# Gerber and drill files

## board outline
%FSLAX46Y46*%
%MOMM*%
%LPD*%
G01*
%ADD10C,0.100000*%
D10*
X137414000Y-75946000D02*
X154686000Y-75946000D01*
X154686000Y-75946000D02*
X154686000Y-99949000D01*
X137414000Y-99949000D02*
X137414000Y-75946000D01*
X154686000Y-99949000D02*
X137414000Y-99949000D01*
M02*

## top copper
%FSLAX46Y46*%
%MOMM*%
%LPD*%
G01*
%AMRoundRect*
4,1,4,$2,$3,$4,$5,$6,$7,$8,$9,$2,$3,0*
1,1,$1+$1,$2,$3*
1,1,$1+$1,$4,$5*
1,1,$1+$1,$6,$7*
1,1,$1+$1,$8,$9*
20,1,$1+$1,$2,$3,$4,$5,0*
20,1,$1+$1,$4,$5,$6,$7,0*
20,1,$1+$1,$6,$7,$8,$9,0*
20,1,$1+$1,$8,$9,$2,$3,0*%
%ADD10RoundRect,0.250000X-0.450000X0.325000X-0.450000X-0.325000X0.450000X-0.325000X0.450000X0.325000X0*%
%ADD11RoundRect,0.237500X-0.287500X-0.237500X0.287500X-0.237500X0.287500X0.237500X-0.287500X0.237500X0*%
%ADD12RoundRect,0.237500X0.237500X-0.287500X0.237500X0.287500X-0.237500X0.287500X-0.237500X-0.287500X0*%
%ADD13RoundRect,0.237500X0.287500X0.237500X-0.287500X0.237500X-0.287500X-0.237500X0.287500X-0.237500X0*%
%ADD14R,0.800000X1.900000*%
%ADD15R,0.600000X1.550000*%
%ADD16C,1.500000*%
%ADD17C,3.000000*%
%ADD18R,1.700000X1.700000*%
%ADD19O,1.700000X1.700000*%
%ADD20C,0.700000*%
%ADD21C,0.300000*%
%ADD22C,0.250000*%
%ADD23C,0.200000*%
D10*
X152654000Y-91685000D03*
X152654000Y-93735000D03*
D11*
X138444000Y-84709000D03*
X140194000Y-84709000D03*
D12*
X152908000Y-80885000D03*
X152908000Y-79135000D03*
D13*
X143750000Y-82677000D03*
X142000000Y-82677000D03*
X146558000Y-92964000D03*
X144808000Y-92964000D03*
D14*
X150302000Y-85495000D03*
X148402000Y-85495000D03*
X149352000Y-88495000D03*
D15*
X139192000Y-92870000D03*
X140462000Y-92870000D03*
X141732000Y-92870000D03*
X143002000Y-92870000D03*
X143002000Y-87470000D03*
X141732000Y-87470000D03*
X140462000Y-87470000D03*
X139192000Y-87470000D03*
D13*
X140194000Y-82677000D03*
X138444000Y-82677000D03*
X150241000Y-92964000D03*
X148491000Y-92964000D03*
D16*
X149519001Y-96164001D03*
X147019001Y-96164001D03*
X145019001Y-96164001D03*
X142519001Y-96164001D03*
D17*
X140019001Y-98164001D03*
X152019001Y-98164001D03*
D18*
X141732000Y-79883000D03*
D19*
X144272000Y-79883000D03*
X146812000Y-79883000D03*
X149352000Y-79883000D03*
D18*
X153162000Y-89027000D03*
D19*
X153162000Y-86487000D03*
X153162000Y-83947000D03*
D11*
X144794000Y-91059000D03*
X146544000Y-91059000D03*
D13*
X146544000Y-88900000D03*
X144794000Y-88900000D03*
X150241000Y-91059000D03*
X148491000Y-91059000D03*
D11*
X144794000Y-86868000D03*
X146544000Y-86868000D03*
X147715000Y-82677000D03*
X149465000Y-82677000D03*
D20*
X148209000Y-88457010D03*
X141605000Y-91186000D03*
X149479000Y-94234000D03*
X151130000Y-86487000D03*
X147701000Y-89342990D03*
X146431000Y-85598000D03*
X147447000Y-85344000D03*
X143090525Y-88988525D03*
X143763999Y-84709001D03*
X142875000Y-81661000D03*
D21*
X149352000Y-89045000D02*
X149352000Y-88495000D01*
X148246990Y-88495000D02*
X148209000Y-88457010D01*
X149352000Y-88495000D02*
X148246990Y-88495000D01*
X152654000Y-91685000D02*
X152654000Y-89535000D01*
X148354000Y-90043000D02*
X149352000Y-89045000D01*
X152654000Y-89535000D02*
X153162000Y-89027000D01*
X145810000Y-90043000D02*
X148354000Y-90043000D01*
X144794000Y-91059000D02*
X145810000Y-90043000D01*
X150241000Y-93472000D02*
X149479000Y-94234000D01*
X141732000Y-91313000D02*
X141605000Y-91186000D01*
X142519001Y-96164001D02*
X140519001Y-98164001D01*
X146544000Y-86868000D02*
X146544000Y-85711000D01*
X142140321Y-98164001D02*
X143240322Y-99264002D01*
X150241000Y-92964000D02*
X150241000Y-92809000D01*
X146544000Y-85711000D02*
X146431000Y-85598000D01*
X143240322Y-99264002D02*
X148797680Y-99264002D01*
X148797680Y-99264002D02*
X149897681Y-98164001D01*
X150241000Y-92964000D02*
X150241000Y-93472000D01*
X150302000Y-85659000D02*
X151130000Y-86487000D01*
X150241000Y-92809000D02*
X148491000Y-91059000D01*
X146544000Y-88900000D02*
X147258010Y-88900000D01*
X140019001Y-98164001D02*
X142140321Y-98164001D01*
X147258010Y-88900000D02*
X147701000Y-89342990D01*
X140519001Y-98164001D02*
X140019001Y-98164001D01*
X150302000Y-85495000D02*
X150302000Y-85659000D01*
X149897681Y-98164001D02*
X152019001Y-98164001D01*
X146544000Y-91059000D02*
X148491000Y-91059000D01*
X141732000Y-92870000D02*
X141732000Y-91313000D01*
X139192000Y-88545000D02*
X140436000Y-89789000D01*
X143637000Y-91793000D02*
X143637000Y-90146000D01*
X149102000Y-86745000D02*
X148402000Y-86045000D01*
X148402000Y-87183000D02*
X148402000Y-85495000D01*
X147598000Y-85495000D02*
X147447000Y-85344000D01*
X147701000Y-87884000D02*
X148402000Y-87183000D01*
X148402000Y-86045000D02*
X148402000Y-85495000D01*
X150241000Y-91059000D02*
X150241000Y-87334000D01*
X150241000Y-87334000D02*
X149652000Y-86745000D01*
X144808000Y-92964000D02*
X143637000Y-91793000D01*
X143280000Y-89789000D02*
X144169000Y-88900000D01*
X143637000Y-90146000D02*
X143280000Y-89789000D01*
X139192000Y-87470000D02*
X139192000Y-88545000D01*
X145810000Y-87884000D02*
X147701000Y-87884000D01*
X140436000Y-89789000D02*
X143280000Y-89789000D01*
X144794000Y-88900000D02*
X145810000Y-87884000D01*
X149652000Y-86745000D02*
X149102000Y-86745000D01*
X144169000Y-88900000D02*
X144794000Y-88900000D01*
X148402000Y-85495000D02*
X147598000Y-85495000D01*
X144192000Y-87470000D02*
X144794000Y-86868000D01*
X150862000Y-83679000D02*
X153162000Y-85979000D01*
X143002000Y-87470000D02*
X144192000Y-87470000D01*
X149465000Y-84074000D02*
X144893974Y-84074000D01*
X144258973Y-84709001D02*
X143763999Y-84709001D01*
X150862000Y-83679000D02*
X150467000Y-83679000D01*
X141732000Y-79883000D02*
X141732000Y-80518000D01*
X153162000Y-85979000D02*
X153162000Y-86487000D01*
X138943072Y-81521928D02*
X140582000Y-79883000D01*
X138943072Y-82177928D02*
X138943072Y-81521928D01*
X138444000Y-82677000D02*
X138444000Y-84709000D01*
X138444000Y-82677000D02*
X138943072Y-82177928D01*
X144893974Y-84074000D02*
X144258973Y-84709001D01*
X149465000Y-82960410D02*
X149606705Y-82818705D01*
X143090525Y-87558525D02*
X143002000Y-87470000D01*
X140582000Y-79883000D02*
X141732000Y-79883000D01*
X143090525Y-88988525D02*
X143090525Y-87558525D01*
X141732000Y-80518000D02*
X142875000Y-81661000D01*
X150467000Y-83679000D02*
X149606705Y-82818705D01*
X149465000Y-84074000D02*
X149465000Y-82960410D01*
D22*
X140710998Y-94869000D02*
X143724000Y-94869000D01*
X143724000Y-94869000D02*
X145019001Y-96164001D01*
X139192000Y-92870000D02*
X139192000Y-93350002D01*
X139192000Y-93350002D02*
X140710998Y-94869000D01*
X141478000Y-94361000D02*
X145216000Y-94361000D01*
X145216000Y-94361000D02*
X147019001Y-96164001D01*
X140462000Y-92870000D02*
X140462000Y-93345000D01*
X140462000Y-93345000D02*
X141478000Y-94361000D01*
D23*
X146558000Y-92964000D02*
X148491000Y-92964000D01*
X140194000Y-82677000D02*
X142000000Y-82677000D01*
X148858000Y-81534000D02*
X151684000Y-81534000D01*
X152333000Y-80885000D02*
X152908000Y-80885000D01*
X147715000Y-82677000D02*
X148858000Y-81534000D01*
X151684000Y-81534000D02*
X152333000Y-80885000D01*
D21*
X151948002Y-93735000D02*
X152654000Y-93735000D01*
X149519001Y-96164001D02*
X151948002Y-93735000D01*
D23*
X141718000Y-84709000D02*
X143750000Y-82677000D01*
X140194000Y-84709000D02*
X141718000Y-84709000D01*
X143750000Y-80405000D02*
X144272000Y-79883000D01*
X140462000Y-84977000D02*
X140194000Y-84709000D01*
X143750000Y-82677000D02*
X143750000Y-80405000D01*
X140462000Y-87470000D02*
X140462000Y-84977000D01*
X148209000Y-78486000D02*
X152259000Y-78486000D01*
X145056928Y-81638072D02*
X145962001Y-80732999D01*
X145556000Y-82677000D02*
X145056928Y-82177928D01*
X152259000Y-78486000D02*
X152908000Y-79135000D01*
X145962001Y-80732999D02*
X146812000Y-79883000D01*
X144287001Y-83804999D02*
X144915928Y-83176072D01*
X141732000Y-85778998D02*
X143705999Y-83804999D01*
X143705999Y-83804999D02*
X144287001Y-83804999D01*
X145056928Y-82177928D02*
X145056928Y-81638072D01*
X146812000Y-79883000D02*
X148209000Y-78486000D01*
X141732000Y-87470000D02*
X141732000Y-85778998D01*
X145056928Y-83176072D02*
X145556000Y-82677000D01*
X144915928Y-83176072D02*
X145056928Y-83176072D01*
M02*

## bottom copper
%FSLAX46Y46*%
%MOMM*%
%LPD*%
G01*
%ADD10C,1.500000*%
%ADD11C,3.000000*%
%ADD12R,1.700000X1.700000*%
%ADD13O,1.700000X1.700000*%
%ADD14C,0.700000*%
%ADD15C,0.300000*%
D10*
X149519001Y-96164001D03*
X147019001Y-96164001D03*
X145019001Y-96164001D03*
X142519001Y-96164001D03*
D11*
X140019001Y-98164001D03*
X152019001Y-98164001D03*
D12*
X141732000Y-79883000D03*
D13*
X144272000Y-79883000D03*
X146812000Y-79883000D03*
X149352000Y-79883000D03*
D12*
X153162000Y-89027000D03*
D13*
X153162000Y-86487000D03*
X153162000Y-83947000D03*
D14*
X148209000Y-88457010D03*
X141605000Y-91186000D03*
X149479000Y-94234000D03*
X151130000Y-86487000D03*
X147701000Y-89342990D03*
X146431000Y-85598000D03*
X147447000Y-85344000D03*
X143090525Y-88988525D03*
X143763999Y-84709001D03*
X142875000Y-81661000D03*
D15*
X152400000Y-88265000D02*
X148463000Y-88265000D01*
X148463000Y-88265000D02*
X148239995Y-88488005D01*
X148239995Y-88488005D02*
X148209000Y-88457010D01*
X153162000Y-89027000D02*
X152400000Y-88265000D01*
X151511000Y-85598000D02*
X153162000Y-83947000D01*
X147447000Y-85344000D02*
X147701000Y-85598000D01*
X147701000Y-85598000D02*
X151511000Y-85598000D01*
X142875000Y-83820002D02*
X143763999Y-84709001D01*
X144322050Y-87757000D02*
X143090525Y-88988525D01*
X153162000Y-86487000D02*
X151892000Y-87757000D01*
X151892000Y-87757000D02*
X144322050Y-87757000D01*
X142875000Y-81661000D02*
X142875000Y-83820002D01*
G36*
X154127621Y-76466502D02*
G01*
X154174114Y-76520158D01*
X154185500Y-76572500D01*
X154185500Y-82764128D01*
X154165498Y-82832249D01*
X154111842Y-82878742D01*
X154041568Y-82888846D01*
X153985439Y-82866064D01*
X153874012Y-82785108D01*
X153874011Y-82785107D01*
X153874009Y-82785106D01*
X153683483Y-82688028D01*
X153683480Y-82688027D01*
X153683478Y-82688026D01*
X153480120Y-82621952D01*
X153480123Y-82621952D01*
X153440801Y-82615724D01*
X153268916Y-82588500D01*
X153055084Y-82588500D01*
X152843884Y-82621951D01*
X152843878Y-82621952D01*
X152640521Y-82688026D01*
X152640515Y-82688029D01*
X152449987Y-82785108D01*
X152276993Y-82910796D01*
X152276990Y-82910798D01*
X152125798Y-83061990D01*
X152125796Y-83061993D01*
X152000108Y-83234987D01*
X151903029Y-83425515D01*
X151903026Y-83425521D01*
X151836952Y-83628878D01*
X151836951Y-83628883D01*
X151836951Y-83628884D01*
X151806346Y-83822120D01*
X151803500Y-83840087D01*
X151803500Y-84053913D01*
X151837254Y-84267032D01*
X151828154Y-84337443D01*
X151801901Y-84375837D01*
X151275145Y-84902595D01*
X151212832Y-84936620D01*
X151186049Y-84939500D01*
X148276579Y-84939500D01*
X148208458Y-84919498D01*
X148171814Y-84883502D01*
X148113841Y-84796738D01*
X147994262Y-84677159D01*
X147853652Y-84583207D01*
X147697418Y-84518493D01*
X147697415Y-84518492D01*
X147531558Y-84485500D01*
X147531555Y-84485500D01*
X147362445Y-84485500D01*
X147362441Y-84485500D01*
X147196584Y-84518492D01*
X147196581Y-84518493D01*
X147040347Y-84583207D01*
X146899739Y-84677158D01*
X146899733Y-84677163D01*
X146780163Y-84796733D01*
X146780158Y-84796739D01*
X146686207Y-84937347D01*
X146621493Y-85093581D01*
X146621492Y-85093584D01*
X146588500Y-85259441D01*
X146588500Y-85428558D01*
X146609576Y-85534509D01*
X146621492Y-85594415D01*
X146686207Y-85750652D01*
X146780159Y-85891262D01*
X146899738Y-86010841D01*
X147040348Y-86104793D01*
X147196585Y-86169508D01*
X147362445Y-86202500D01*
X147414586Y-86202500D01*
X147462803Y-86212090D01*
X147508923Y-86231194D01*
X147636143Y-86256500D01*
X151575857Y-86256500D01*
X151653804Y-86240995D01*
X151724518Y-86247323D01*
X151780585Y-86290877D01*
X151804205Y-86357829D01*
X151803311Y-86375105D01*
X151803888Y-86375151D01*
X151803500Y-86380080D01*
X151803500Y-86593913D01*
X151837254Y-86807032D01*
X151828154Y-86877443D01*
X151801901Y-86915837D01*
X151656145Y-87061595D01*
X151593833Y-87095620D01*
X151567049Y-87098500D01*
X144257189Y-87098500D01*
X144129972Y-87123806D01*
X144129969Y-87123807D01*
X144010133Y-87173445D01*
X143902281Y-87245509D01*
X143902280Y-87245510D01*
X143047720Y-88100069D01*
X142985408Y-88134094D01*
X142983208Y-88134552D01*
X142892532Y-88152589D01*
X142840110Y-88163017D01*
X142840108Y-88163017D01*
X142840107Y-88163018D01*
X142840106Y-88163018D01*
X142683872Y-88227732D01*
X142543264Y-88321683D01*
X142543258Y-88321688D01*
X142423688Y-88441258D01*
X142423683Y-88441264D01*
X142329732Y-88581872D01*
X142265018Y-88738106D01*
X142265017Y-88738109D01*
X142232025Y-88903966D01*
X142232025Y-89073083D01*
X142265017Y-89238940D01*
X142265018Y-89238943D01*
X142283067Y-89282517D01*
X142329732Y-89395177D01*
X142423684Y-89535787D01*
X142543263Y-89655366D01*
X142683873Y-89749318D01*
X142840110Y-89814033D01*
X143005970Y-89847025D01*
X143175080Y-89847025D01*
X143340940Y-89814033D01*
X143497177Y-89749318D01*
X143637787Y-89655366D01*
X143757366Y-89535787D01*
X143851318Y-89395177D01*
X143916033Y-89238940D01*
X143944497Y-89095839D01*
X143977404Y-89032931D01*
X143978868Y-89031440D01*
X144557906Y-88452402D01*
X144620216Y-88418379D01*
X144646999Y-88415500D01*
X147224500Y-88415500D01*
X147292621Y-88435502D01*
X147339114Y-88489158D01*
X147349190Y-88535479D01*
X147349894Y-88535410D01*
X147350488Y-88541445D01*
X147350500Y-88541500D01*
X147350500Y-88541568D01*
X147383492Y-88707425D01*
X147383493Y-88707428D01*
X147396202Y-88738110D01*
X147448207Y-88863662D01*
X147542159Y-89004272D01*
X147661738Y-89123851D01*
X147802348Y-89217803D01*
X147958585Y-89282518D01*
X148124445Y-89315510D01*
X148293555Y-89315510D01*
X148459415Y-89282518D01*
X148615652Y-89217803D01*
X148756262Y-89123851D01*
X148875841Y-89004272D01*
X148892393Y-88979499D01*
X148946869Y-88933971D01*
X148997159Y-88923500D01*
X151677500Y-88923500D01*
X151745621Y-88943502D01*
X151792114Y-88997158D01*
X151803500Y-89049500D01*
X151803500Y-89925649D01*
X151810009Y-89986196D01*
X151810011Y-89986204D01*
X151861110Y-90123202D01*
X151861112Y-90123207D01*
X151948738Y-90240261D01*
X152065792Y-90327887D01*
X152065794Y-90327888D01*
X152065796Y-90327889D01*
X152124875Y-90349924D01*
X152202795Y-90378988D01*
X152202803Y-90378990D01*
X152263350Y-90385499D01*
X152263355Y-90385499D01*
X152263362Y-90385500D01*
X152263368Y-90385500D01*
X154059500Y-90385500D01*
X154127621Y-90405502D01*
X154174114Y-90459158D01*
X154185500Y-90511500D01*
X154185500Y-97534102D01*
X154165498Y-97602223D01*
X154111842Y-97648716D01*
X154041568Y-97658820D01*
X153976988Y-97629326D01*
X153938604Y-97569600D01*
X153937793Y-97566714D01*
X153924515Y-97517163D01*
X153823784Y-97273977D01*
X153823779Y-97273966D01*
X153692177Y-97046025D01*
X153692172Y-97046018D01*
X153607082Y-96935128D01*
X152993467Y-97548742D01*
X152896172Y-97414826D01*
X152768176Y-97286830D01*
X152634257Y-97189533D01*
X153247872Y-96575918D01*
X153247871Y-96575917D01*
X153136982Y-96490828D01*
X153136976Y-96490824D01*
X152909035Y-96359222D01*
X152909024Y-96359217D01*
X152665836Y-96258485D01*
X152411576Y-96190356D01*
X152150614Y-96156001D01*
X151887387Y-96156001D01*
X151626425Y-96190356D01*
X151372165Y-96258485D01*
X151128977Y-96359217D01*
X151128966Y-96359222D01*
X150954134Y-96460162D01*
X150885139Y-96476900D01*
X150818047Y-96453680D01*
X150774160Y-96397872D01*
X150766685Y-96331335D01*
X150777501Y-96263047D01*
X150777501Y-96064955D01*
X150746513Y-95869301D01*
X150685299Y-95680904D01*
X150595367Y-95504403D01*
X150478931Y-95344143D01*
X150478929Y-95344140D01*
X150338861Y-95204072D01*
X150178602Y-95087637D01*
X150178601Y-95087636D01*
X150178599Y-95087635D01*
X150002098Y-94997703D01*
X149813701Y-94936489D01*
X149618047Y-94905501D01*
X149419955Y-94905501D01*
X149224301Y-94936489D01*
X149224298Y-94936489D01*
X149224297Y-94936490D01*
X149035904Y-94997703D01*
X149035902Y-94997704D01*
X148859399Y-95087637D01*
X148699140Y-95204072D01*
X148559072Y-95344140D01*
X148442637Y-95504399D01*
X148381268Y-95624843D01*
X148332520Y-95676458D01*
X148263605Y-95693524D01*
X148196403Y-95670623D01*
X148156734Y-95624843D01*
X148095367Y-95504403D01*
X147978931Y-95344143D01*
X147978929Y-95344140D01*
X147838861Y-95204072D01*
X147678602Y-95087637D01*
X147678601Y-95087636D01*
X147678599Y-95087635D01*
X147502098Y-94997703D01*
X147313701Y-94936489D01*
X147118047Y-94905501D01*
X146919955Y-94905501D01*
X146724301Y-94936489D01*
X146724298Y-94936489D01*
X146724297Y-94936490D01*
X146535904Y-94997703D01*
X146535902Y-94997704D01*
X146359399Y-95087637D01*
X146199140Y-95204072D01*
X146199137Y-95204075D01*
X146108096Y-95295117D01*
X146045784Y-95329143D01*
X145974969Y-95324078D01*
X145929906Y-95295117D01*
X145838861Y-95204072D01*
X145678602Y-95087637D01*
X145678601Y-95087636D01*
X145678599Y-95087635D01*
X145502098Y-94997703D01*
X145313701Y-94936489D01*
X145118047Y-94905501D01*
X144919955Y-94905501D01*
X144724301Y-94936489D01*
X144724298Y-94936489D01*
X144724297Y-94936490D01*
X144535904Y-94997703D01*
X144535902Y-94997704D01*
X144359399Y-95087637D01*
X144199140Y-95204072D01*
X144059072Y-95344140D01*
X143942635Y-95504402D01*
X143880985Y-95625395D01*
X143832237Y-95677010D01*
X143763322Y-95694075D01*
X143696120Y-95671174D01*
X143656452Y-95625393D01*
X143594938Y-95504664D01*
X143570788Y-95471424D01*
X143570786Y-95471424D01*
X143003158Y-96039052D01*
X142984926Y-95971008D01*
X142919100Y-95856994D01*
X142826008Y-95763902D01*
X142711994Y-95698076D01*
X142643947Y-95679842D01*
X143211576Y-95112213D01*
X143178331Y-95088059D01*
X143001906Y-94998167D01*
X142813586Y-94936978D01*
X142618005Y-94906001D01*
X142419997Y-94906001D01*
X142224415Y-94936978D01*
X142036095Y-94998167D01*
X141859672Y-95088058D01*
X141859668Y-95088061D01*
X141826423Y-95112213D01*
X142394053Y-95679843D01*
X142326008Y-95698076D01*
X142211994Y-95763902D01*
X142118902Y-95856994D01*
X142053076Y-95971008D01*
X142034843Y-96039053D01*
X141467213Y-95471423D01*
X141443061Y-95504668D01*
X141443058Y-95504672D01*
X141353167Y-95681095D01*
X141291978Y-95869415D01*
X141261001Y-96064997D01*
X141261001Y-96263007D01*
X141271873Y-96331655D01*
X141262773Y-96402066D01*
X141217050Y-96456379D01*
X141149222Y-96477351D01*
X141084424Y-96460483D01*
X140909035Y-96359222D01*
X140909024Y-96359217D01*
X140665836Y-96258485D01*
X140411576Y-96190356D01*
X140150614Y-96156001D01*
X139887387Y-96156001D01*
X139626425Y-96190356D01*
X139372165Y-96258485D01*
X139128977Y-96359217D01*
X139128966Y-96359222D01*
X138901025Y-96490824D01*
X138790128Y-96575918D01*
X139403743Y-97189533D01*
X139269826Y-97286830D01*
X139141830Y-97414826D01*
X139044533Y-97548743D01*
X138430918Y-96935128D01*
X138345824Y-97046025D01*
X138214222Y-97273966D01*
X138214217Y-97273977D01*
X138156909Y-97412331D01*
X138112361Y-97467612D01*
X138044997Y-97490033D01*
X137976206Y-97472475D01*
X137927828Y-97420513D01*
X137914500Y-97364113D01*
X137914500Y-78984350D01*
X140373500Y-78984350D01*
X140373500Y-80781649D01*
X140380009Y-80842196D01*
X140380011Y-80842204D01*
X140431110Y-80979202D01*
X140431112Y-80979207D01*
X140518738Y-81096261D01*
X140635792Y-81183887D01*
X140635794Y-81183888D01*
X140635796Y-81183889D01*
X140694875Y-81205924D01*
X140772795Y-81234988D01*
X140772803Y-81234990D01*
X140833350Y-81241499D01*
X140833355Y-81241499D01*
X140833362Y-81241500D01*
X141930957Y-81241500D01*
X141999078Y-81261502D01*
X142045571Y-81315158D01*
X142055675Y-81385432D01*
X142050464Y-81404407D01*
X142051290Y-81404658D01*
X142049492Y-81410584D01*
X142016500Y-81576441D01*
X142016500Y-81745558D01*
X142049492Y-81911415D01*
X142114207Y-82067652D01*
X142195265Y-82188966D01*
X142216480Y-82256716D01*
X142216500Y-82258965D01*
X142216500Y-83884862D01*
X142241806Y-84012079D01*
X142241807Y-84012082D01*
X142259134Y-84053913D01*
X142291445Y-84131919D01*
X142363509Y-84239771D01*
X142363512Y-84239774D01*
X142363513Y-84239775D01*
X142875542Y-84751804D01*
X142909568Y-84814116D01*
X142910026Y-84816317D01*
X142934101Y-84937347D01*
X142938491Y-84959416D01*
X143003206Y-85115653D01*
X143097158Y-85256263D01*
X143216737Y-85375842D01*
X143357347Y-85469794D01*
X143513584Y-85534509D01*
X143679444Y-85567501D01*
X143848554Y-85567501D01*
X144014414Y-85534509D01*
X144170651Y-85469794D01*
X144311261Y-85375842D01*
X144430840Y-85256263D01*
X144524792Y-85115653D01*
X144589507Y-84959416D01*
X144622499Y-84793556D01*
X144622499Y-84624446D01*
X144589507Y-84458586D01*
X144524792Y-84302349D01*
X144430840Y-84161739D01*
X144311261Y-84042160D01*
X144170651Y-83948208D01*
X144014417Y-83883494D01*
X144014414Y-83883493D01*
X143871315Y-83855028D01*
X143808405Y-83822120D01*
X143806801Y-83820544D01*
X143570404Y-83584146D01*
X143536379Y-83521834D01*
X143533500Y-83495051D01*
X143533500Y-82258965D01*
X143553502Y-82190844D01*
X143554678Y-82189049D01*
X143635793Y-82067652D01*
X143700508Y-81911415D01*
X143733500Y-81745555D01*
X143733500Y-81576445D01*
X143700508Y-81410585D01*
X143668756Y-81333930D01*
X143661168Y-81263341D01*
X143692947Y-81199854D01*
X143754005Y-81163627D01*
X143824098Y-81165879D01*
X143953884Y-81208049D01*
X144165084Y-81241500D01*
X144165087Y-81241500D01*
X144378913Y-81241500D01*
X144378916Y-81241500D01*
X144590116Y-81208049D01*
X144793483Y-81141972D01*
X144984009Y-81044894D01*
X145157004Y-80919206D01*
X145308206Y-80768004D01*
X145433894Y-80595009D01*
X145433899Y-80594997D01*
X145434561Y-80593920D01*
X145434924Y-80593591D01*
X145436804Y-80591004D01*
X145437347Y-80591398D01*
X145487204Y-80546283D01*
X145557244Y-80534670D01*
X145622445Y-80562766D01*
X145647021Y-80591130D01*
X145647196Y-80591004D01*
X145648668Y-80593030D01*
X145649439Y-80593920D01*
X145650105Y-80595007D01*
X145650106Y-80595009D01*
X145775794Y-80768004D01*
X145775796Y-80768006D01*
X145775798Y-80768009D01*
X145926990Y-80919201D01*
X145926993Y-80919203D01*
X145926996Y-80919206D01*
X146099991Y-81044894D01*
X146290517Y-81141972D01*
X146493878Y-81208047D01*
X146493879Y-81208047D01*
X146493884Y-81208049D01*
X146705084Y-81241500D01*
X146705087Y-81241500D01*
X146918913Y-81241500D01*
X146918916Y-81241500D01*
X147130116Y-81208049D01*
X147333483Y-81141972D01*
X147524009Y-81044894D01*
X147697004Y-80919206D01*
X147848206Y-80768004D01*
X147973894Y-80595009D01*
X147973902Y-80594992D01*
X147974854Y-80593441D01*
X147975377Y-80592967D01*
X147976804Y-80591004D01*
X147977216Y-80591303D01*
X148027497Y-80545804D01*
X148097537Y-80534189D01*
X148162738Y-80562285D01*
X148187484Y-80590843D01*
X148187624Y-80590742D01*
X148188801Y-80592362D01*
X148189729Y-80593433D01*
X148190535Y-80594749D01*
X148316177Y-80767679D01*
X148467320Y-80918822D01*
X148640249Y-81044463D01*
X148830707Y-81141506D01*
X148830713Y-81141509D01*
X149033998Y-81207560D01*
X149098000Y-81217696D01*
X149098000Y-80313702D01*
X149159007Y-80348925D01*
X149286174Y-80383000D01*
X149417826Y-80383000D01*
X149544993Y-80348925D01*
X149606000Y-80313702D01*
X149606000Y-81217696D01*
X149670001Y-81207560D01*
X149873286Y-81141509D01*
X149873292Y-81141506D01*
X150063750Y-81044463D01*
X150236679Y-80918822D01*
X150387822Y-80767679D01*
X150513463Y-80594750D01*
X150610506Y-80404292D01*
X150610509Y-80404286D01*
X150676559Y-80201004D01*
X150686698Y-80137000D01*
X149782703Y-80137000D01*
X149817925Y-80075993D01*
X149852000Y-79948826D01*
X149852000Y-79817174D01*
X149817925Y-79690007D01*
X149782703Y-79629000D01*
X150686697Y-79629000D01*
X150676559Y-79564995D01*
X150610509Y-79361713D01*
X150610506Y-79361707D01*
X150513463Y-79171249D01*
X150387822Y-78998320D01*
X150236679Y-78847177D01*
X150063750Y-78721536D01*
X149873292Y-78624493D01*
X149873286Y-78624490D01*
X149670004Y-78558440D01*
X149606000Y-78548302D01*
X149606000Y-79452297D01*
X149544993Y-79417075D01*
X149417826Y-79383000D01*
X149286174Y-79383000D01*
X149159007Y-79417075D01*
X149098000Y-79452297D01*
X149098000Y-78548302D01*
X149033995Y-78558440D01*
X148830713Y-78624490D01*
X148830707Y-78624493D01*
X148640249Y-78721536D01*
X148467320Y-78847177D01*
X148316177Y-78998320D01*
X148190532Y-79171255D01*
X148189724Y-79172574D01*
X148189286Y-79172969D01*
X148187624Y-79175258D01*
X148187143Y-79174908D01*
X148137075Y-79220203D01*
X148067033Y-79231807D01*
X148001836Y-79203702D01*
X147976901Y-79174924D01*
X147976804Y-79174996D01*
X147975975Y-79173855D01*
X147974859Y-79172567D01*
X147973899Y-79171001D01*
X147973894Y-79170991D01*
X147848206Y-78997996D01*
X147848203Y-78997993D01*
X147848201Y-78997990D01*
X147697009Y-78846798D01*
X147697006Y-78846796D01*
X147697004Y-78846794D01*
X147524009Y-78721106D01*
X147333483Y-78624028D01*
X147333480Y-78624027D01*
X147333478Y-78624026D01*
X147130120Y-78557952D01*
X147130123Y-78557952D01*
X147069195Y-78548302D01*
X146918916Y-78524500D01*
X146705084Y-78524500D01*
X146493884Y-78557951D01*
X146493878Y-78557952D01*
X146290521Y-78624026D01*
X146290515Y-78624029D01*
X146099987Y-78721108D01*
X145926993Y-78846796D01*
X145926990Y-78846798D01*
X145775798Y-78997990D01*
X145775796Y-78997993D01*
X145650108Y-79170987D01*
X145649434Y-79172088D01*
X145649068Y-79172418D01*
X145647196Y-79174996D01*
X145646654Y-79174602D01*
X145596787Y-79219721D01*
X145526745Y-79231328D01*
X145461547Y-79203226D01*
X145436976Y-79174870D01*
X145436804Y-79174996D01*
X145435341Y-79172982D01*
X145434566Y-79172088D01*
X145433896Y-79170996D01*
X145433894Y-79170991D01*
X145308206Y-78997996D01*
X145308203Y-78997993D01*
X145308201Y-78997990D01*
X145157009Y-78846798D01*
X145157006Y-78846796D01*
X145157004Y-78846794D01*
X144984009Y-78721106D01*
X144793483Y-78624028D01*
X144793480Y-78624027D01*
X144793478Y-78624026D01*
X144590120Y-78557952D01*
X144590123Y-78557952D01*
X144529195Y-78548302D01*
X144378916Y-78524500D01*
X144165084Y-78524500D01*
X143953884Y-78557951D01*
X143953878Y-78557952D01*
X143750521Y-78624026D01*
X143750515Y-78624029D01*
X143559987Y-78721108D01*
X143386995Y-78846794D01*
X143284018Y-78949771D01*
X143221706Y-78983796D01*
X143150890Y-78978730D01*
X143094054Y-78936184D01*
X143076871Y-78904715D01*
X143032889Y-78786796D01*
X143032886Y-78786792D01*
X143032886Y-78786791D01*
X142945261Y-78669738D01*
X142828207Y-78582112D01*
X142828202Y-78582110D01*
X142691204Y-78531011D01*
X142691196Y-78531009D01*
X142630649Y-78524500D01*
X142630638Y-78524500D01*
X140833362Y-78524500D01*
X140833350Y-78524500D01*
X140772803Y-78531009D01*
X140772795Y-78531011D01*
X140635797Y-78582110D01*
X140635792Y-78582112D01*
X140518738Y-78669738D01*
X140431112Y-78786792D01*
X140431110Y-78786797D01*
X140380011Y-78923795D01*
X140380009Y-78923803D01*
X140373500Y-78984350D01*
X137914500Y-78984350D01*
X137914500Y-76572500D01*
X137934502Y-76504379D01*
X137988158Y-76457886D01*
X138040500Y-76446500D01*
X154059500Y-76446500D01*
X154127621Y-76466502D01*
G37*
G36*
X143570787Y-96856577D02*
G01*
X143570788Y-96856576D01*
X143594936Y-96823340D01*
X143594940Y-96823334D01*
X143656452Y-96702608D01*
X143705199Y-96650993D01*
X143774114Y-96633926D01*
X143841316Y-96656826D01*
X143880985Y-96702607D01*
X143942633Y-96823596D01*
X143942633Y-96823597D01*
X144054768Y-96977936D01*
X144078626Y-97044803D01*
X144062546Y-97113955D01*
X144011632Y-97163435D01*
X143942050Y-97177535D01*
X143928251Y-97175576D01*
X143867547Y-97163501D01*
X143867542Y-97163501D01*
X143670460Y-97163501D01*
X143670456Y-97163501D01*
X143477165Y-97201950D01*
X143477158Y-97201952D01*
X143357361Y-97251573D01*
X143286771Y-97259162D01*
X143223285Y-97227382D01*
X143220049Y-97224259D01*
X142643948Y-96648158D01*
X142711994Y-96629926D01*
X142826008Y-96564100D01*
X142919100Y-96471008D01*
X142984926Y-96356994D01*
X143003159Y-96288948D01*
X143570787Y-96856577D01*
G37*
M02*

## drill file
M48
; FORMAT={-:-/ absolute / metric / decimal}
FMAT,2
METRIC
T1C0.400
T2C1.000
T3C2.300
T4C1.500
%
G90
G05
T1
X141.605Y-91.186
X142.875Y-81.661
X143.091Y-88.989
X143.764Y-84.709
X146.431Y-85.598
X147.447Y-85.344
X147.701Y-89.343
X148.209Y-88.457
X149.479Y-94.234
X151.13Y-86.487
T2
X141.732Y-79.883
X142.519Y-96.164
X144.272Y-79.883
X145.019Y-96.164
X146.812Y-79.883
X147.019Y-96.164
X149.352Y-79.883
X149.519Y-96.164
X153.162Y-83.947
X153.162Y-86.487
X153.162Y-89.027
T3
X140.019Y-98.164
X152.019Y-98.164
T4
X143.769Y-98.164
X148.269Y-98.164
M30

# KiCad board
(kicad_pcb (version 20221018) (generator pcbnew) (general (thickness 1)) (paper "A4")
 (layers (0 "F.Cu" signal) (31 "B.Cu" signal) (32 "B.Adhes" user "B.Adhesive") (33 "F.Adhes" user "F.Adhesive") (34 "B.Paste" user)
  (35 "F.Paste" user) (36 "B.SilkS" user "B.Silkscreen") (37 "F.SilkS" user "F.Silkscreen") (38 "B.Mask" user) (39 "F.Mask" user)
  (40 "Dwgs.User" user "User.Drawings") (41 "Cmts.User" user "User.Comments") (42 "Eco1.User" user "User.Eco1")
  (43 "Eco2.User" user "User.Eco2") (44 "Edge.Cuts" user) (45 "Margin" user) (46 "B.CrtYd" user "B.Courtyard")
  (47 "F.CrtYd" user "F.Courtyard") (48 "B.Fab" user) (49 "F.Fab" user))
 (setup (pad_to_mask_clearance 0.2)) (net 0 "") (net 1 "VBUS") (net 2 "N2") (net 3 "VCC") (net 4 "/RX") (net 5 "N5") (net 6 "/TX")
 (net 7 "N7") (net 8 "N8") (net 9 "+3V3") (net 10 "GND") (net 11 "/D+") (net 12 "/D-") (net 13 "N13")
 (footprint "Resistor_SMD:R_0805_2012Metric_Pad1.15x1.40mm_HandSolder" (layer "F.Cu") (at 152.654 92.71 -90)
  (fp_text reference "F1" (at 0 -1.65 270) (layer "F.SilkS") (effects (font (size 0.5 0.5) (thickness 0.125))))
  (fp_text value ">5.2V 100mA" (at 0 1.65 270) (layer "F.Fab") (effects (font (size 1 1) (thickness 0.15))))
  (pad "1" smd roundrect (at -1.025 0 270) (size 1.15 1.4) (layers "F.Cu" "F.Paste" "F.Mask") (roundrect_rratio 0.217391) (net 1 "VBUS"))
  (pad "2" smd roundrect (at 1.025 0 270) (size 1.15 1.4) (layers "F.Cu" "F.Paste" "F.Mask") (roundrect_rratio 0.217391) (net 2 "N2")))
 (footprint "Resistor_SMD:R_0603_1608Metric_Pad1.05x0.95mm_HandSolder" (layer "F.Cu") (at 139.319 84.709)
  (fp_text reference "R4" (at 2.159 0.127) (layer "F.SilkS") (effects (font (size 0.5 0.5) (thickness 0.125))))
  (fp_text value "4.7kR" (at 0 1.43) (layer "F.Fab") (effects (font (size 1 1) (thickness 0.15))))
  (pad "1" smd roundrect (at -0.875 0) (size 1.05 0.95) (layers "F.Cu" "F.Paste" "F.Mask") (roundrect_rratio 0.25) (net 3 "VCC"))
  (pad "2" smd roundrect (at 0.875 0) (size 1.05 0.95) (layers "F.Cu" "F.Paste" "F.Mask") (roundrect_rratio 0.25) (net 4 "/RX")))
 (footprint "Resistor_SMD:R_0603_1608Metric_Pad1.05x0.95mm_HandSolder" (layer "F.Cu") (at 152.908 80.01 90)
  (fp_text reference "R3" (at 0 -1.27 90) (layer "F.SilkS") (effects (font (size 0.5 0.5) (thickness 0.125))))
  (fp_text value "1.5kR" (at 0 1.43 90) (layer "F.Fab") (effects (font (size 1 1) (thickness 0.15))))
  (pad "1" smd roundrect (at -0.875 0 90) (size 1.05 0.95) (layers "F.Cu" "F.Paste" "F.Mask") (roundrect_rratio 0.25) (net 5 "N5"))
  (pad "2" smd roundrect (at 0.875 0 90) (size 1.05 0.95) (layers "F.Cu" "F.Paste" "F.Mask") (roundrect_rratio 0.25) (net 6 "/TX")))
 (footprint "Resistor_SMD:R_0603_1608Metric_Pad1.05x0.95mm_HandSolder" (layer "F.Cu") (at 142.875 82.677 180)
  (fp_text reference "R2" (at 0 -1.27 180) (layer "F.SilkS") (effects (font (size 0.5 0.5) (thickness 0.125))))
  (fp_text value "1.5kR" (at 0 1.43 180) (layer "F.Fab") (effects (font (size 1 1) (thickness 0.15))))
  (pad "1" smd roundrect (at -0.875 0 180) (size 1.05 0.95) (layers "F.Cu" "F.Paste" "F.Mask") (roundrect_rratio 0.25) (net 4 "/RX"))
  (pad "2" smd roundrect (at 0.875 0 180) (size 1.05 0.95) (layers "F.Cu" "F.Paste" "F.Mask") (roundrect_rratio 0.25) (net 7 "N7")))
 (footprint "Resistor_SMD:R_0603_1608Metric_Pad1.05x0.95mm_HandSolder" (layer "F.Cu") (at 145.683 92.964 180)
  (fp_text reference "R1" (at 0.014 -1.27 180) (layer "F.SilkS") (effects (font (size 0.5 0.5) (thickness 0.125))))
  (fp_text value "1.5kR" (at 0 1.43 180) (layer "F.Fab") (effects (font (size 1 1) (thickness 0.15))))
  (pad "1" smd roundrect (at -0.875 0 180) (size 1.05 0.95) (layers "F.Cu" "F.Paste" "F.Mask") (roundrect_rratio 0.25) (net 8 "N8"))
  (pad "2" smd roundrect (at 0.875 0 180) (size 1.05 0.95) (layers "F.Cu" "F.Paste" "F.Mask") (roundrect_rratio 0.25) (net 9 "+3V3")))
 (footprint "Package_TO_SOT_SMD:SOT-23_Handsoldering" (layer "F.Cu") (at 149.352 86.995 -90)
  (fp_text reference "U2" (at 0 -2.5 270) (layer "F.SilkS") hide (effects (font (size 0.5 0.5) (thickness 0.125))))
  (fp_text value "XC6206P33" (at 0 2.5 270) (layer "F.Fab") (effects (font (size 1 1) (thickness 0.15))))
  (pad "1" smd rect (at -1.5 -0.95 270) (size 1.9 0.8) (layers "F.Cu" "F.Paste" "F.Mask") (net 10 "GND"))
  (pad "2" smd rect (at -1.5 0.95 270) (size 1.9 0.8) (layers "F.Cu" "F.Paste" "F.Mask") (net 9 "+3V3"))
  (pad "3" smd rect (at 1.5 0 270) (size 1.9 0.8) (layers "F.Cu" "F.Paste" "F.Mask") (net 1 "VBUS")))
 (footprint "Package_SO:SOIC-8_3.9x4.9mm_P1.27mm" (layer "F.Cu") (at 141.097 90.17 90)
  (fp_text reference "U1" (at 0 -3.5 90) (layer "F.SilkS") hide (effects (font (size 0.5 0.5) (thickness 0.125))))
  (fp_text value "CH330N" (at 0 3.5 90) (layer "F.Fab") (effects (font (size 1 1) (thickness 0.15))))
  (pad "1" smd rect (at -2.7 -1.905 90) (size 1.55 0.6) (layers "F.Cu" "F.Paste" "F.Mask") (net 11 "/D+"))
  (pad "2" smd rect (at -2.7 -0.635 90) (size 1.55 0.6) (layers "F.Cu" "F.Paste" "F.Mask") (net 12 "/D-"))
  (pad "3" smd rect (at -2.7 0.635 90) (size 1.55 0.6) (layers "F.Cu" "F.Paste" "F.Mask") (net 10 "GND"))
  (pad "4" smd rect (at -2.7 1.905 90) (size 1.55 0.6) (layers "F.Cu" "F.Paste" "F.Mask") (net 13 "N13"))
  (pad "5" smd rect (at 2.7 1.905 90) (size 1.55 0.6) (layers "F.Cu" "F.Paste" "F.Mask") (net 3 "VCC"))
  (pad "6" smd rect (at 2.7 0.635 90) (size 1.55 0.6) (layers "F.Cu" "F.Paste" "F.Mask") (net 6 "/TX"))
  (pad "7" smd rect (at 2.7 -0.635 90) (size 1.55 0.6) (layers "F.Cu" "F.Paste" "F.Mask") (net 4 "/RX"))
  (pad "8" smd rect (at 2.7 -1.905 90) (size 1.55 0.6) (layers "F.Cu" "F.Paste" "F.Mask") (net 9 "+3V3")))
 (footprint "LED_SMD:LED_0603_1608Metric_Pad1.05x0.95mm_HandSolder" (layer "F.Cu") (at 139.319 82.677 180)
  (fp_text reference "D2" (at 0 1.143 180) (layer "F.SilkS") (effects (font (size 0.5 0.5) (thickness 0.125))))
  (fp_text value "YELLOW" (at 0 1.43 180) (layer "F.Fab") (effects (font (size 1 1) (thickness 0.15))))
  (pad "1" smd roundrect (at -0.875 0 180) (size 1.05 0.95) (layers "F.Cu" "F.Paste" "F.Mask") (roundrect_rratio 0.25) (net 7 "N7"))
  (pad "2" smd roundrect (at 0.875 0 180) (size 1.05 0.95) (layers "F.Cu" "F.Paste" "F.Mask") (roundrect_rratio 0.25) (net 3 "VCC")))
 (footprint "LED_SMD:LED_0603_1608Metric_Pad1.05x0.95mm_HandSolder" (layer "F.Cu") (at 149.366 92.964 180)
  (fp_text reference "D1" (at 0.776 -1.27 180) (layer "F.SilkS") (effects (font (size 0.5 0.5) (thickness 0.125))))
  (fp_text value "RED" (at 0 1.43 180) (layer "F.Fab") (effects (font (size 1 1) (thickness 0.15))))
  (pad "1" smd roundrect (at -0.875 0 180) (size 1.05 0.95) (layers "F.Cu" "F.Paste" "F.Mask") (roundrect_rratio 0.25) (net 10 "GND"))
  (pad "2" smd roundrect (at 0.875 0 180) (size 1.05 0.95) (layers "F.Cu" "F.Paste" "F.Mask") (roundrect_rratio 0.25) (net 8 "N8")))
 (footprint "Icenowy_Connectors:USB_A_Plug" (layer "F.Cu") (at 142.519001 96.164001)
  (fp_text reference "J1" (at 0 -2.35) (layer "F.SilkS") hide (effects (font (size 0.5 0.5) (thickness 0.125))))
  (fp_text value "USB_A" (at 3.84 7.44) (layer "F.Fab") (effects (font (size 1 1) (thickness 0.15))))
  (pad "" np_thru_hole circle (at 1.25 2 270) (size 1.5 1.5) (drill 1.5) (layers "*.Cu" "*.Mask"))
  (pad "" np_thru_hole circle (at 5.75 2 270) (size 1.5 1.5) (drill 1.5) (layers "*.Cu" "*.Mask"))
  (pad "1" thru_hole circle (at 7 0 270) (size 1.5 1.5) (drill 1) (layers "*.Cu" "*.Mask") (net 2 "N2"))
  (pad "2" thru_hole circle (at 4.5 0 270) (size 1.5 1.5) (drill 1) (layers "*.Cu" "*.Mask") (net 12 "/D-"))
  (pad "3" thru_hole circle (at 2.5 0 270) (size 1.5 1.5) (drill 1) (layers "*.Cu" "*.Mask") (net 11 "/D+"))
  (pad "4" thru_hole circle (at 0 0 270) (size 1.5 1.5) (drill 1) (layers "*.Cu" "*.Mask") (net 10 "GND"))
  (pad "5" thru_hole circle (at -2.5 2 270) (size 3 3) (drill 2.3) (layers "*.Cu" "*.Mask") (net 10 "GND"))
  (pad "5" thru_hole circle (at 9.5 2 270) (size 3 3) (drill 2.3) (layers "*.Cu" "*.Mask") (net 10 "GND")))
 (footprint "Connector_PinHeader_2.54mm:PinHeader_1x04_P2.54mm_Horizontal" (layer "F.Cu") (at 141.732 79.883 90)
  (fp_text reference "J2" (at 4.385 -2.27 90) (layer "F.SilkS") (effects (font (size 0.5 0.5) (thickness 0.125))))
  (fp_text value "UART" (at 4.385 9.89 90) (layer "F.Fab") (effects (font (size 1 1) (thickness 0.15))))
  (pad "1" thru_hole rect (at 0 0 90) (size 1.7 1.7) (drill 1) (layers "*.Cu" "*.Mask") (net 3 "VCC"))
  (pad "2" thru_hole oval (at 0 2.54 90) (size 1.7 1.7) (drill 1) (layers "*.Cu" "*.Mask") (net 4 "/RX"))
  (pad "3" thru_hole oval (at 0 5.08 90) (size 1.7 1.7) (drill 1) (layers "*.Cu" "*.Mask") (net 6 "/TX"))
  (pad "4" thru_hole oval (at 0 7.62 90) (size 1.7 1.7) (drill 1) (layers "*.Cu" "*.Mask") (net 10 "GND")))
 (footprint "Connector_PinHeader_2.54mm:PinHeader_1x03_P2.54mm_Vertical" (layer "F.Cu") (at 153.162 89.027 180)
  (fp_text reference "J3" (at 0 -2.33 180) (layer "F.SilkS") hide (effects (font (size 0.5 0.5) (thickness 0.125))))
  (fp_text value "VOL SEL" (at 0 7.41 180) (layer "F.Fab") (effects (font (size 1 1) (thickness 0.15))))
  (pad "1" thru_hole rect (at 0 0 180) (size 1.7 1.7) (drill 1) (layers "*.Cu" "*.Mask") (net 1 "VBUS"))
  (pad "2" thru_hole oval (at 0 2.54 180) (size 1.7 1.7) (drill 1) (layers "*.Cu" "*.Mask") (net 3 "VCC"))
  (pad "3" thru_hole oval (at 0 5.08 180) (size 1.7 1.7) (drill 1) (layers "*.Cu" "*.Mask") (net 9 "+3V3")))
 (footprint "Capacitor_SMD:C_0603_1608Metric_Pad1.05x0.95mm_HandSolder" (layer "F.Cu") (at 145.669 91.059)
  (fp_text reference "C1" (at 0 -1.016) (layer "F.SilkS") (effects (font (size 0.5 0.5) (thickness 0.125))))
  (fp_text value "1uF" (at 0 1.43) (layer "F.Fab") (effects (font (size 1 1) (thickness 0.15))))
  (pad "1" smd roundrect (at -0.875 0) (size 1.05 0.95) (layers "F.Cu" "F.Paste" "F.Mask") (roundrect_rratio 0.25) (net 1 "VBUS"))
  (pad "2" smd roundrect (at 0.875 0) (size 1.05 0.95) (layers "F.Cu" "F.Paste" "F.Mask") (roundrect_rratio 0.25) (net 10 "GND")))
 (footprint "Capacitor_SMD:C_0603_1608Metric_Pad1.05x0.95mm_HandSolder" (layer "F.Cu") (at 145.669 88.9 180)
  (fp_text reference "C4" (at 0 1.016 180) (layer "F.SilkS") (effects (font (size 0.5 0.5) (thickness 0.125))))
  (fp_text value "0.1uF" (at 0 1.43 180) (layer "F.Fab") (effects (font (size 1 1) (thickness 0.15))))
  (pad "1" smd roundrect (at -0.875 0 180) (size 1.05 0.95) (layers "F.Cu" "F.Paste" "F.Mask") (roundrect_rratio 0.25) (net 10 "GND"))
  (pad "2" smd roundrect (at 0.875 0 180) (size 1.05 0.95) (layers "F.Cu" "F.Paste" "F.Mask") (roundrect_rratio 0.25) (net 9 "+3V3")))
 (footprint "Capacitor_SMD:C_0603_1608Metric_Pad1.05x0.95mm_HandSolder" (layer "F.Cu") (at 149.366 91.059 180)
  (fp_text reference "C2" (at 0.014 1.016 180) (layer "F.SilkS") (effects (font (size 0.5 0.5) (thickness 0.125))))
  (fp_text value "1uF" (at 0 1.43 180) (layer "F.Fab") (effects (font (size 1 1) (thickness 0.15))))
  (pad "1" smd roundrect (at -0.875 0 180) (size 1.05 0.95) (layers "F.Cu" "F.Paste" "F.Mask") (roundrect_rratio 0.25) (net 9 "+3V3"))
  (pad "2" smd roundrect (at 0.875 0 180) (size 1.05 0.95) (layers "F.Cu" "F.Paste" "F.Mask") (roundrect_rratio 0.25) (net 10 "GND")))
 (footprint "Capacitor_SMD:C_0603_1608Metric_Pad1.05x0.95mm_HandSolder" (layer "F.Cu") (at 145.669 86.868)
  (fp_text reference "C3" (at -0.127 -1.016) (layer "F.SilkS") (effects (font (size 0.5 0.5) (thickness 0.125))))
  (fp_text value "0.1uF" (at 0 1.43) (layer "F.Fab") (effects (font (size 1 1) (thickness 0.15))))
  (pad "1" smd roundrect (at -0.875 0) (size 1.05 0.95) (layers "F.Cu" "F.Paste" "F.Mask") (roundrect_rratio 0.25) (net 3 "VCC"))
  (pad "2" smd roundrect (at 0.875 0) (size 1.05 0.95) (layers "F.Cu" "F.Paste" "F.Mask") (roundrect_rratio 0.25) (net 10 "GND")))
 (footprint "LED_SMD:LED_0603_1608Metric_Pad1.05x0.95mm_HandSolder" (layer "F.Cu") (at 148.59 82.677)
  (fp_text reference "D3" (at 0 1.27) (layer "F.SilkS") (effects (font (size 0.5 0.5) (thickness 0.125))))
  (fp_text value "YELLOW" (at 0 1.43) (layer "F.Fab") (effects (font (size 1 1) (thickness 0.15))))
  (pad "1" smd roundrect (at -0.875 0) (size 1.05 0.95) (layers "F.Cu" "F.Paste" "F.Mask") (roundrect_rratio 0.25) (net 5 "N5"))
  (pad "2" smd roundrect (at 0.875 0) (size 1.05 0.95) (layers "F.Cu" "F.Paste" "F.Mask") (roundrect_rratio 0.25) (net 3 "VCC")))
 (gr_line (start 137.414 75.946) (end 154.686 75.946) (stroke (width 0.1) (type solid)) (layer "Edge.Cuts"))
 (gr_line (start 154.686 75.946) (end 154.686 99.949) (stroke (width 0.1) (type solid)) (layer "Edge.Cuts"))
 (gr_line (start 137.414 99.949) (end 137.414 75.946) (stroke (width 0.1) (type solid)) (layer "Edge.Cuts"))
 (gr_line (start 154.686 99.949) (end 137.414 99.949) (stroke (width 0.1) (type solid)) (layer "Edge.Cuts"))
 (segment (start 149.352 89.045) (end 149.352 88.495) (width 0.3) (layer "F.Cu") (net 1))
 (segment (start 148.24699 88.495) (end 148.209 88.45701) (width 0.3) (layer "F.Cu") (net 1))
 (segment (start 149.352 88.495) (end 148.24699 88.495) (width 0.3) (layer "F.Cu") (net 1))
 (segment (start 152.654 91.685) (end 152.654 89.535) (width 0.3) (layer "F.Cu") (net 1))
 (segment (start 148.354 90.043) (end 149.352 89.045) (width 0.3) (layer "F.Cu") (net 1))
 (segment (start 152.654 89.535) (end 153.162 89.027) (width 0.3) (layer "F.Cu") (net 1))
 (segment (start 145.81 90.043) (end 148.354 90.043) (width 0.3) (layer "F.Cu") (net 1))
 (segment (start 144.794 91.059) (end 145.81 90.043) (width 0.3) (layer "F.Cu") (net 1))
 (via (at 148.209 88.45701) (size 0.7) (drill 0.4) (layers "F.Cu" "B.Cu") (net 1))
 (segment (start 152.4 88.265) (end 148.463 88.265) (width 0.3) (layer "B.Cu") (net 1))
 (segment (start 148.463 88.265) (end 148.239995 88.488005) (width 0.3) (layer "B.Cu") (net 1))
 (segment (start 148.239995 88.488005) (end 148.209 88.45701) (width 0.3) (layer "B.Cu") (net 1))
 (segment (start 153.162 89.027) (end 152.4 88.265) (width 0.3) (layer "B.Cu") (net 1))
 (segment (start 150.241 93.472) (end 149.479 94.234) (width 0.3) (layer "F.Cu") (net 10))
 (segment (start 141.732 91.313) (end 141.605 91.186) (width 0.3) (layer "F.Cu") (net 10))
 (segment (start 142.519001 96.164001) (end 140.519001 98.164001) (width 0.3) (layer "F.Cu") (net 10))
 (segment (start 146.544 86.868) (end 146.544 85.711) (width 0.3) (layer "F.Cu") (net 10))
 (segment (start 142.140321 98.164001) (end 143.240322 99.264002) (width 0.3) (layer "F.Cu") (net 10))
 (segment (start 150.241 92.964) (end 150.241 92.809) (width 0.3) (layer "F.Cu") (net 10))
 (segment (start 146.544 85.711) (end 146.431 85.598) (width 0.3) (layer "F.Cu") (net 10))
 (segment (start 143.240322 99.264002) (end 148.79768 99.264002) (width 0.3) (layer "F.Cu") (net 10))
 (segment (start 148.79768 99.264002) (end 149.897681 98.164001) (width 0.3) (layer "F.Cu") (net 10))
 (segment (start 150.241 92.964) (end 150.241 93.472) (width 0.3) (layer "F.Cu") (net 10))
 (segment (start 150.302 85.659) (end 151.13 86.487) (width 0.3) (layer "F.Cu") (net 10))
 (segment (start 150.241 92.809) (end 148.491 91.059) (width 0.3) (layer "F.Cu") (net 10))
 (segment (start 146.544 88.9) (end 147.25801 88.9) (width 0.3) (layer "F.Cu") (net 10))
 (segment (start 140.019001 98.164001) (end 142.140321 98.164001) (width 0.3) (layer "F.Cu") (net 10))
 (segment (start 147.25801 88.9) (end 147.701 89.34299) (width 0.3) (layer "F.Cu") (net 10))
 (segment (start 140.519001 98.164001) (end 140.019001 98.164001) (width 0.3) (layer "F.Cu") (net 10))
 (segment (start 150.302 85.495) (end 150.302 85.659) (width 0.3) (layer "F.Cu") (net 10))
 (segment (start 149.897681 98.164001) (end 152.019001 98.164001) (width 0.3) (layer "F.Cu") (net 10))
 (segment (start 146.544 91.059) (end 148.491 91.059) (width 0.3) (layer "F.Cu") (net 10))
 (segment (start 141.732 92.87) (end 141.732 91.313) (width 0.3) (layer "F.Cu") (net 10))
 (via (at 141.605 91.186) (size 0.7) (drill 0.4) (layers "F.Cu" "B.Cu") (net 10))
 (via (at 149.479 94.234) (size 0.7) (drill 0.4) (layers "F.Cu" "B.Cu") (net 10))
 (via (at 151.13 86.487) (size 0.7) (drill 0.4) (layers "F.Cu" "B.Cu") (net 10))
 (via (at 147.701 89.34299) (size 0.7) (drill 0.4) (layers "F.Cu" "B.Cu") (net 10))
 (via (at 146.431 85.598) (size 0.7) (drill 0.4) (layers "F.Cu" "B.Cu") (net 10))
 (segment (start 139.192 88.545) (end 140.436 89.789) (width 0.3) (layer "F.Cu") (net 9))
 (segment (start 143.637 91.793) (end 143.637 90.146) (width 0.3) (layer "F.Cu") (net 9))
 (segment (start 149.102 86.745) (end 148.402 86.045) (width 0.3) (layer "F.Cu") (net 9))
 (segment (start 148.402 87.183) (end 148.402 85.495) (width 0.3) (layer "F.Cu") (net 9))
 (segment (start 147.598 85.495) (end 147.447 85.344) (width 0.3) (layer "F.Cu") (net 9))
 (segment (start 147.701 87.884) (end 148.402 87.183) (width 0.3) (layer "F.Cu") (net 9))
 (segment (start 148.402 86.045) (end 148.402 85.495) (width 0.3) (layer "F.Cu") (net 9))
 (segment (start 150.241 91.059) (end 150.241 87.334) (width 0.3) (layer "F.Cu") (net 9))
 (segment (start 150.241 87.334) (end 149.652 86.745) (width 0.3) (layer "F.Cu") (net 9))
 (segment (start 144.808 92.964) (end 143.637 91.793) (width 0.3) (layer "F.Cu") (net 9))
 (segment (start 143.28 89.789) (end 144.169 88.9) (width 0.3) (layer "F.Cu") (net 9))
 (segment (start 143.637 90.146) (end 143.28 89.789) (width 0.3) (layer "F.Cu") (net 9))
 (segment (start 139.192 87.47) (end 139.192 88.545) (width 0.3) (layer "F.Cu") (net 9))
 (segment (start 145.81 87.884) (end 147.701 87.884) (width 0.3) (layer "F.Cu") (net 9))
 (segment (start 140.436 89.789) (end 143.28 89.789) (width 0.3) (layer "F.Cu") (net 9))
 (segment (start 144.794 88.9) (end 145.81 87.884) (width 0.3) (layer "F.Cu") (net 9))
 (segment (start 149.652 86.745) (end 149.102 86.745) (width 0.3) (layer "F.Cu") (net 9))
 (segment (start 144.169 88.9) (end 144.794 88.9) (width 0.3) (layer "F.Cu") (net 9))
 (segment (start 148.402 85.495) (end 147.598 85.495) (width 0.3) (layer "F.Cu") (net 9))
 (via (at 147.447 85.344) (size 0.7) (drill 0.4) (layers "F.Cu" "B.Cu") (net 9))
 (segment (start 151.511 85.598) (end 153.162 83.947) (width 0.3) (layer "B.Cu") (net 9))
 (segment (start 147.447 85.344) (end 147.701 85.598) (width 0.3) (layer "B.Cu") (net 9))
 (segment (start 147.701 85.598) (end 151.511 85.598) (width 0.3) (layer "B.Cu") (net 9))
 (segment (start 144.192 87.47) (end 144.794 86.868) (width 0.3) (layer "F.Cu") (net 3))
 (segment (start 150.862 83.679) (end 153.162 85.979) (width 0.3) (layer "F.Cu") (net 3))
 (segment (start 143.002 87.47) (end 144.192 87.47) (width 0.3) (layer "F.Cu") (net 3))
 (segment (start 149.465 84.074) (end 144.893974 84.074) (width 0.3) (layer "F.Cu") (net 3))
 (segment (start 144.258973 84.709001) (end 143.763999 84.709001) (width 0.3) (layer "F.Cu") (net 3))
 (segment (start 150.862 83.679) (end 150.467 83.679) (width 0.3) (layer "F.Cu") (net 3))
 (segment (start 141.732 79.883) (end 141.732 80.518) (width 0.3) (layer "F.Cu") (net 3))
 (segment (start 153.162 85.979) (end 153.162 86.487) (width 0.3) (layer "F.Cu") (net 3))
 (segment (start 138.943072 81.521928) (end 140.582 79.883) (width 0.3) (layer "F.Cu") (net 3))
 (segment (start 138.943072 82.177928) (end 138.943072 81.521928) (width 0.3) (layer "F.Cu") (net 3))
 (segment (start 138.444 82.677) (end 138.444 84.709) (width 0.3) (layer "F.Cu") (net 3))
 (segment (start 138.444 82.677) (end 138.943072 82.177928) (width 0.3) (layer "F.Cu") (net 3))
 (segment (start 144.893974 84.074) (end 144.258973 84.709001) (width 0.3) (layer "F.Cu") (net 3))
 (segment (start 149.465 82.96041) (end 149.606705 82.818705) (width 0.3) (layer "F.Cu") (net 3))
 (segment (start 143.090525 87.558525) (end 143.002 87.47) (width 0.3) (layer "F.Cu") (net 3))
 (segment (start 140.582 79.883) (end 141.732 79.883) (width 0.3) (layer "F.Cu") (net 3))
 (segment (start 143.090525 88.988525) (end 143.090525 87.558525) (width 0.3) (layer "F.Cu") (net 3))
 (segment (start 141.732 80.518) (end 142.875 81.661) (width 0.3) (layer "F.Cu") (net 3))
 (segment (start 150.467 83.679) (end 149.606705 82.818705) (width 0.3) (layer "F.Cu") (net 3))
 (segment (start 149.465 84.074) (end 149.465 82.96041) (width 0.3) (layer "F.Cu") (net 3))
 (via (at 143.090525 88.988525) (size 0.7) (drill 0.4) (layers "F.Cu" "B.Cu") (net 3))
 (via (at 143.763999 84.709001) (size 0.7) (drill 0.4) (layers "F.Cu" "B.Cu") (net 3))
 (via (at 142.875 81.661) (size 0.7) (drill 0.4) (layers "F.Cu" "B.Cu") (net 3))
 (segment (start 142.875 83.820002) (end 143.763999 84.709001) (width 0.3) (layer "B.Cu") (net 3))
 (segment (start 144.32205 87.757) (end 143.090525 88.988525) (width 0.3) (layer "B.Cu") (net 3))
 (segment (start 153.162 86.487) (end 151.892 87.757) (width 0.3) (layer "B.Cu") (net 3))
 (segment (start 151.892 87.757) (end 144.32205 87.757) (width 0.3) (layer "B.Cu") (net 3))
 (segment (start 142.875 81.661) (end 142.875 83.820002) (width 0.3) (layer "B.Cu") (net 3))
 (segment (start 140.710998 94.869) (end 143.724 94.869) (width 0.25) (layer "F.Cu") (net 11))
 (segment (start 143.724 94.869) (end 145.019001 96.164001) (width 0.25) (layer "F.Cu") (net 11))
 (segment (start 139.192 92.87) (end 139.192 93.350002) (width 0.25) (layer "F.Cu") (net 11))
 (segment (start 139.192 93.350002) (end 140.710998 94.869) (width 0.25) (layer "F.Cu") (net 11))
 (segment (start 141.478 94.361) (end 145.216 94.361) (width 0.25) (layer "F.Cu") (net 12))
 (segment (start 145.216 94.361) (end 147.019001 96.164001) (width 0.25) (layer "F.Cu") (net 12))
 (segment (start 140.462 92.87) (end 140.462 93.345) (width 0.25) (layer "F.Cu") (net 12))
 (segment (start 140.462 93.345) (end 141.478 94.361) (width 0.25) (layer "F.Cu") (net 12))
 (segment (start 146.558 92.964) (end 148.491 92.964) (width 0.2) (layer "F.Cu") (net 8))
 (segment (start 140.194 82.677) (end 142 82.677) (width 0.2) (layer "F.Cu") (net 7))
 (segment (start 148.858 81.534) (end 151.684 81.534) (width 0.2) (layer "F.Cu") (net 5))
 (segment (start 152.333 80.885) (end 152.908 80.885) (width 0.2) (layer "F.Cu") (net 5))
 (segment (start 147.715 82.677) (end 148.858 81.534) (width 0.2) (layer "F.Cu") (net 5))
 (segment (start 151.684 81.534) (end 152.333 80.885) (width 0.2) (layer "F.Cu") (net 5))
 (segment (start 151.948002 93.735) (end 152.654 93.735) (width 0.3) (layer "F.Cu") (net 2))
 (segment (start 149.519001 96.164001) (end 151.948002 93.735) (width 0.3) (layer "F.Cu") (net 2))
 (segment (start 141.718 84.709) (end 143.75 82.677) (width 0.2) (layer "F.Cu") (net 4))
 (segment (start 140.194 84.709) (end 141.718 84.709) (width 0.2) (layer "F.Cu") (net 4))
 (segment (start 143.75 80.405) (end 144.272 79.883) (width 0.2) (layer "F.Cu") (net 4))
 (segment (start 140.462 84.977) (end 140.194 84.709) (width 0.2) (layer "F.Cu") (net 4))
 (segment (start 143.75 82.677) (end 143.75 80.405) (width 0.2) (layer "F.Cu") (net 4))
 (segment (start 140.462 87.47) (end 140.462 84.977) (width 0.2) (layer "F.Cu") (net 4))
 (segment (start 148.209 78.486) (end 152.259 78.486) (width 0.2) (layer "F.Cu") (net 6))
 (segment (start 145.056928 81.638072) (end 145.962001 80.732999) (width 0.2) (layer "F.Cu") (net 6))
 (segment (start 145.556 82.677) (end 145.056928 82.177928) (width 0.2) (layer "F.Cu") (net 6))
 (segment (start 152.259 78.486) (end 152.908 79.135) (width 0.2) (layer "F.Cu") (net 6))
 (segment (start 145.962001 80.732999) (end 146.812 79.883) (width 0.2) (layer "F.Cu") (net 6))
 (segment (start 144.287001 83.804999) (end 144.915928 83.176072) (width 0.2) (layer "F.Cu") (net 6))
 (segment (start 141.732 85.778998) (end 143.705999 83.804999) (width 0.2) (layer "F.Cu") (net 6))
 (segment (start 143.705999 83.804999) (end 144.287001 83.804999) (width 0.2) (layer "F.Cu") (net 6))
 (segment (start 145.056928 82.177928) (end 145.056928 81.638072) (width 0.2) (layer "F.Cu") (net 6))
 (segment (start 146.812 79.883) (end 148.209 78.486) (width 0.2) (layer "F.Cu") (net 6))
 (segment (start 141.732 87.47) (end 141.732 85.778998) (width 0.2) (layer "F.Cu") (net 6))
 (segment (start 145.056928 83.176072) (end 145.556 82.677) (width 0.2) (layer "F.Cu") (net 6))
 (segment (start 144.915928 83.176072) (end 145.056928 83.176072) (width 0.2) (layer "F.Cu") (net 6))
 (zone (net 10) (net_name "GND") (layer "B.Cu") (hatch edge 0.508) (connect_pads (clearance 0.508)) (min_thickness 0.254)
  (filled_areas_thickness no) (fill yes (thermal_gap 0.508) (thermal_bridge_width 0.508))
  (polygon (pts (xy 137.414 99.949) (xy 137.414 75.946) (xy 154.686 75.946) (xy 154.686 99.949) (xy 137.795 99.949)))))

